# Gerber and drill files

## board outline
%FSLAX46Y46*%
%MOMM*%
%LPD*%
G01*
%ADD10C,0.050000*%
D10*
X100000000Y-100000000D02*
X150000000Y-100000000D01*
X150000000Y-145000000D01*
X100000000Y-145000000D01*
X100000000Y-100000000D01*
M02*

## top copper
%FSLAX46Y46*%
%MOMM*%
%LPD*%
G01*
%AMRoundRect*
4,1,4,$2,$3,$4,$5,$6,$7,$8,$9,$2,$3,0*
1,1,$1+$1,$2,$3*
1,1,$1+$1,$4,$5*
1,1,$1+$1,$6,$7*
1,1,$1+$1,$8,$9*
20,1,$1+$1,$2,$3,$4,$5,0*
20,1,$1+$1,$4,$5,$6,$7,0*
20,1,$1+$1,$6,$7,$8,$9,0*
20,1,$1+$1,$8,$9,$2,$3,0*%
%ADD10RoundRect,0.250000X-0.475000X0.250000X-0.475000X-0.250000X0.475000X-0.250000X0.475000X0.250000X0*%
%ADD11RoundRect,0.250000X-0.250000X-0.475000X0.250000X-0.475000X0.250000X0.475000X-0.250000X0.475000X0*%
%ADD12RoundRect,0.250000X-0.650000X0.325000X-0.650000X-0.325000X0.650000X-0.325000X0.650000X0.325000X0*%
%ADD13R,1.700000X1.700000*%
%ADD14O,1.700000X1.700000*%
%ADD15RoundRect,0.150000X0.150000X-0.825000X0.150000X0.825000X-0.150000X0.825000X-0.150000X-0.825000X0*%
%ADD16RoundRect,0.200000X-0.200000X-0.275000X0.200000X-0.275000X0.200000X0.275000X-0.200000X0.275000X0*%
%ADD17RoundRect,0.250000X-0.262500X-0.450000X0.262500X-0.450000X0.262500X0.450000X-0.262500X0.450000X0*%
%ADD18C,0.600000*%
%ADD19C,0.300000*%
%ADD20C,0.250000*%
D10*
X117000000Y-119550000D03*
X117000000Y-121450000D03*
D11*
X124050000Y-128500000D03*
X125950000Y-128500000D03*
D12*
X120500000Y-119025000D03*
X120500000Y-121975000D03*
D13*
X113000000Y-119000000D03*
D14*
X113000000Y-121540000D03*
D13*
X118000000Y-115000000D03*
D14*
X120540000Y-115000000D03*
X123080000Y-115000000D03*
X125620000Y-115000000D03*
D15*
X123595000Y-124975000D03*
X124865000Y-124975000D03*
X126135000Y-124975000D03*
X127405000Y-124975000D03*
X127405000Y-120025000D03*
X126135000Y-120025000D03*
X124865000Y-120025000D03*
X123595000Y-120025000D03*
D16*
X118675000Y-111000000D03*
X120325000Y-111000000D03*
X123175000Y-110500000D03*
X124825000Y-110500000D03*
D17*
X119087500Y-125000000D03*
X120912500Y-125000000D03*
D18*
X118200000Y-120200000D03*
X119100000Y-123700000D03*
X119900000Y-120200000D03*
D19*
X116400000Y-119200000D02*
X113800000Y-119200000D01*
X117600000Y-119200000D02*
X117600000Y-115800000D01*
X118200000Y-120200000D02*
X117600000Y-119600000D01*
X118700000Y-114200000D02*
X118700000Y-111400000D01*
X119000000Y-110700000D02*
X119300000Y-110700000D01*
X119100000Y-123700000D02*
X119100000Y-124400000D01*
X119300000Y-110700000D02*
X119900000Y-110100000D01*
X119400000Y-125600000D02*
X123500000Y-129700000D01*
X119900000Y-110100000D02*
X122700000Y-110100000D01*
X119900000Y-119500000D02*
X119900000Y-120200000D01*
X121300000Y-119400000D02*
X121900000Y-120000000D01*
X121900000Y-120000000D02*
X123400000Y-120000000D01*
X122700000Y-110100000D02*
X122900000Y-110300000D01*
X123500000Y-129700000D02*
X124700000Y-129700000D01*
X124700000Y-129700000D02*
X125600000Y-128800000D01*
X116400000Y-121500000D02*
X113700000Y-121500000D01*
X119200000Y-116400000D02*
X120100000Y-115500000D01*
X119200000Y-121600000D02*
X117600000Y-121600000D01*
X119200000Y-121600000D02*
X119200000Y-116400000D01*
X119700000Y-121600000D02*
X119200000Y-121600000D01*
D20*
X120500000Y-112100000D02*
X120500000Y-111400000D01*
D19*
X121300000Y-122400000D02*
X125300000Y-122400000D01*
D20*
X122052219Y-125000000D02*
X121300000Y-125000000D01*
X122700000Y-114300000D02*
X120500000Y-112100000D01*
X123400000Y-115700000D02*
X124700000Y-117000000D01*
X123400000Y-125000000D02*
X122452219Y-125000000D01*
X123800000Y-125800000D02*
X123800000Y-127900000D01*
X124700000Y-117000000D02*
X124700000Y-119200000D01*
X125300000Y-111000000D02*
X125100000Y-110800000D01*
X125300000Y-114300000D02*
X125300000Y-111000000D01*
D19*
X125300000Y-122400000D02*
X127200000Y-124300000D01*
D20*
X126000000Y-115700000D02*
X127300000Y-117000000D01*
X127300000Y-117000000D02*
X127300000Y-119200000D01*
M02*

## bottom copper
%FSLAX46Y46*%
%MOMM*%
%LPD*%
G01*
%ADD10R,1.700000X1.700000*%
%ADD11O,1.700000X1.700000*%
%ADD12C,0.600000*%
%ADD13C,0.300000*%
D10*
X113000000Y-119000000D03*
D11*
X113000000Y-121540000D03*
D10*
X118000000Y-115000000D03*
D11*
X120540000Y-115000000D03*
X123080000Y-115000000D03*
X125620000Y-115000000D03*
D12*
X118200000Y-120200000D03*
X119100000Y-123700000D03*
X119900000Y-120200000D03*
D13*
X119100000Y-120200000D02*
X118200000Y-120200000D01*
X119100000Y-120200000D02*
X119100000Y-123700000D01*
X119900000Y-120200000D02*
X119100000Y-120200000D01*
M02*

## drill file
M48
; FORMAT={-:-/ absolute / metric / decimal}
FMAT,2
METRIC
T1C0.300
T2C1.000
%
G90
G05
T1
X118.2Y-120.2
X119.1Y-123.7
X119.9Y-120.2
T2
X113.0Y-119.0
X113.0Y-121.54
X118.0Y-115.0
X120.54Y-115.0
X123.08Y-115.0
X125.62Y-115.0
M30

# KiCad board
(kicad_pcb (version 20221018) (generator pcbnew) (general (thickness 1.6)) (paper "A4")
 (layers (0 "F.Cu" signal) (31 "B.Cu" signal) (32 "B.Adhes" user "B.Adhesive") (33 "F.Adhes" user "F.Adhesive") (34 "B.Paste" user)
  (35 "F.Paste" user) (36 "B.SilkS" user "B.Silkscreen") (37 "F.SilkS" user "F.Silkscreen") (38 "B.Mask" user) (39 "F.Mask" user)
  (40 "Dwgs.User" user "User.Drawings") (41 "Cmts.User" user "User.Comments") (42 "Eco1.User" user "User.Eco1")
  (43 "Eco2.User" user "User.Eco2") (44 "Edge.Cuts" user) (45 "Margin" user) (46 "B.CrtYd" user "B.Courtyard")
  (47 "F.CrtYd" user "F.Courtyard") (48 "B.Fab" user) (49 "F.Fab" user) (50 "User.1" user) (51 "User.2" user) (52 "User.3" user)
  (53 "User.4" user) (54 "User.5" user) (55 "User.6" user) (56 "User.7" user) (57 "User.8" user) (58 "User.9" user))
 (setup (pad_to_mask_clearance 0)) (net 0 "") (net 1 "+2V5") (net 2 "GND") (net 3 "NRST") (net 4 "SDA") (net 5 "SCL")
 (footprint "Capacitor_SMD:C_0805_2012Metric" (layer "F.Cu") (at 117 120.5 -90)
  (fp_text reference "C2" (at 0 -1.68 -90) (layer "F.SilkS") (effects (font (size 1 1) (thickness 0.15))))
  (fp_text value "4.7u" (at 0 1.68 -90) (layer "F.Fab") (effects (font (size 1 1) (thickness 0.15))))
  (pad "1" smd roundrect (at -0.95 0 270) (size 1 1.45) (layers "F.Cu" "F.Paste" "F.Mask") (roundrect_rratio 0.25) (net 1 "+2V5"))
  (pad "2" smd roundrect (at 0.95 0 270) (size 1 1.45) (layers "F.Cu" "F.Paste" "F.Mask") (roundrect_rratio 0.25) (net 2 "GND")))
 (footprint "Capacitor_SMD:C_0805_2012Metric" (layer "F.Cu") (at 125 128.5)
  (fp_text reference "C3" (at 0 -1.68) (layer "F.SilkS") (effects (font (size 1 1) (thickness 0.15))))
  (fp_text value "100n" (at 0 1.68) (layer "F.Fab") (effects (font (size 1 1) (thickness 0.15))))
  (pad "1" smd roundrect (at -0.95 0) (size 1 1.45) (layers "F.Cu" "F.Paste" "F.Mask") (roundrect_rratio 0.25) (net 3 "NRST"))
  (pad "2" smd roundrect (at 0.95 0) (size 1 1.45) (layers "F.Cu" "F.Paste" "F.Mask") (roundrect_rratio 0.25) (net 1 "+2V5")))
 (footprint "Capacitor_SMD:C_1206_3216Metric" (layer "F.Cu") (at 120.5 120.5 -90)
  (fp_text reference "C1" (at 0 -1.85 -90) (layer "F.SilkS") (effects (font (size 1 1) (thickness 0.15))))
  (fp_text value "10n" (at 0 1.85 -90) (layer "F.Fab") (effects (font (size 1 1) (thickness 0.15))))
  (pad "1" smd roundrect (at -1.475 0 270) (size 1.15 1.8) (layers "F.Cu" "F.Paste" "F.Mask") (roundrect_rratio 0.217391) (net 1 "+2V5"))
  (pad "2" smd roundrect (at 1.475 0 270) (size 1.15 1.8) (layers "F.Cu" "F.Paste" "F.Mask") (roundrect_rratio 0.217391) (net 2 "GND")))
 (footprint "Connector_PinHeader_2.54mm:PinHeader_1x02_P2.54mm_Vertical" (layer "F.Cu") (at 113 119)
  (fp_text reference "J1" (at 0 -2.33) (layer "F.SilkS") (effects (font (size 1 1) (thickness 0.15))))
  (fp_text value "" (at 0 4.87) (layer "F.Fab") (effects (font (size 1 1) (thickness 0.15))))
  (pad "1" thru_hole rect (at 0 0) (size 1.7 1.7) (drill 1) (layers "*.Cu" "*.Mask") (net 1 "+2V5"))
  (pad "2" thru_hole oval (at 0 2.54) (size 1.7 1.7) (drill 1) (layers "*.Cu" "*.Mask") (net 2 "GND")))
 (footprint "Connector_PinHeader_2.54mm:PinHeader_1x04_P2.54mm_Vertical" (layer "F.Cu") (at 118 115 90)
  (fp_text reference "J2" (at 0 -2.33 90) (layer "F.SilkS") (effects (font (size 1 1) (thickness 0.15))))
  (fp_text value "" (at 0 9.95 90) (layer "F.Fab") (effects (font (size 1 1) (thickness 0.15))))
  (pad "1" thru_hole rect (at 0 0 90) (size 1.7 1.7) (drill 1) (layers "*.Cu" "*.Mask") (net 1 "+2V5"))
  (pad "2" thru_hole oval (at 0 2.54 90) (size 1.7 1.7) (drill 1) (layers "*.Cu" "*.Mask") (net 2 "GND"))
  (pad "3" thru_hole oval (at 0 5.08 90) (size 1.7 1.7) (drill 1) (layers "*.Cu" "*.Mask") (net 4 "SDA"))
  (pad "4" thru_hole oval (at 0 7.62 90) (size 1.7 1.7) (drill 1) (layers "*.Cu" "*.Mask") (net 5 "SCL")))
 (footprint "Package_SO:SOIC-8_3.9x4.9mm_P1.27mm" (layer "F.Cu") (at 125.5 122.5 90)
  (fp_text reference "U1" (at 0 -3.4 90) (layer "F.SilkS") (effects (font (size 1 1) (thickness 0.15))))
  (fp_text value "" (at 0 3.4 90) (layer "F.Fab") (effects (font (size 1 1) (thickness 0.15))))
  (pad "1" smd roundrect (at -2.475 -1.905 90) (size 1.95 0.6) (layers "F.Cu" "F.Paste" "F.Mask") (roundrect_rratio 0.25) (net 3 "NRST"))
  (pad "2" smd roundrect (at -2.475 -0.635 90) (size 1.95 0.6) (layers "F.Cu" "F.Paste" "F.Mask") (roundrect_rratio 0.25))
  (pad "3" smd roundrect (at -2.475 0.635 90) (size 1.95 0.6) (layers "F.Cu" "F.Paste" "F.Mask") (roundrect_rratio 0.25))
  (pad "4" smd roundrect (at -2.475 1.905 90) (size 1.95 0.6) (layers "F.Cu" "F.Paste" "F.Mask") (roundrect_rratio 0.25) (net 2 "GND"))
  (pad "5" smd roundrect (at 2.475 1.905 90) (size 1.95 0.6) (layers "F.Cu" "F.Paste" "F.Mask") (roundrect_rratio 0.25) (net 5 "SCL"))
  (pad "6" smd roundrect (at 2.475 0.635 90) (size 1.95 0.6) (layers "F.Cu" "F.Paste" "F.Mask") (roundrect_rratio 0.25))
  (pad "7" smd roundrect (at 2.475 -0.635 90) (size 1.95 0.6) (layers "F.Cu" "F.Paste" "F.Mask") (roundrect_rratio 0.25) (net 4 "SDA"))
  (pad "8" smd roundrect (at 2.475 -1.905 90) (size 1.95 0.6) (layers "F.Cu" "F.Paste" "F.Mask") (roundrect_rratio 0.25) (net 1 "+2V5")))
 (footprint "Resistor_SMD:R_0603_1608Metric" (layer "F.Cu") (at 119.5 111)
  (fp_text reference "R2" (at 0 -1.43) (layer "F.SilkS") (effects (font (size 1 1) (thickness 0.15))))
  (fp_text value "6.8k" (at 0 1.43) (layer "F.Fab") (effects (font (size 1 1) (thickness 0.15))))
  (pad "1" smd roundrect (at -0.825 0) (size 0.8 0.95) (layers "F.Cu" "F.Paste" "F.Mask") (roundrect_rratio 0.25) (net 1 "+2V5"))
  (pad "2" smd roundrect (at 0.825 0) (size 0.8 0.95) (layers "F.Cu" "F.Paste" "F.Mask") (roundrect_rratio 0.25) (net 4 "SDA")))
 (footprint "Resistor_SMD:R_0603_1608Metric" (layer "F.Cu") (at 124 110.5)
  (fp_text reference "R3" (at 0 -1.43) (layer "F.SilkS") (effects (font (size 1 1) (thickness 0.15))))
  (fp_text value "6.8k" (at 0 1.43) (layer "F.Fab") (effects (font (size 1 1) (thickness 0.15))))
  (pad "1" smd roundrect (at -0.825 0) (size 0.8 0.95) (layers "F.Cu" "F.Paste" "F.Mask") (roundrect_rratio 0.25) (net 1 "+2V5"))
  (pad "2" smd roundrect (at 0.825 0) (size 0.8 0.95) (layers "F.Cu" "F.Paste" "F.Mask") (roundrect_rratio 0.25) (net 5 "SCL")))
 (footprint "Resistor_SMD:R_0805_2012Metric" (layer "F.Cu") (at 120 125)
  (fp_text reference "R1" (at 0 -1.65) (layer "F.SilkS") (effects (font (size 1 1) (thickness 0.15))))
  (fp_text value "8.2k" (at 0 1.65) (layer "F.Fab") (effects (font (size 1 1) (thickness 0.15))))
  (pad "1" smd roundrect (at -0.9125 0) (size 1.025 1.4) (layers "F.Cu" "F.Paste" "F.Mask") (roundrect_rratio 0.243902) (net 1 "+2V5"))
  (pad "2" smd roundrect (at 0.9125 0) (size 1.025 1.4) (layers "F.Cu" "F.Paste" "F.Mask") (roundrect_rratio 0.243902) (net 3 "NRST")))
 (gr_rect (start 100 100) (end 150 145) (stroke (width 0.05) (type default)) (fill none) (layer "Edge.Cuts"))
 (segment (start 116.4 119.2) (end 113.8 119.2) (width 0.3) (layer "F.Cu") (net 1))
 (segment (start 117.6 119.2) (end 117.6 115.8) (width 0.3) (layer "F.Cu") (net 1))
 (segment (start 118.2 120.2) (end 117.6 119.6) (width 0.3) (layer "F.Cu") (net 1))
 (segment (start 118.7 114.2) (end 118.7 111.4) (width 0.3) (layer "F.Cu") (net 1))
 (segment (start 119 110.7) (end 119.3 110.7) (width 0.3) (layer "F.Cu") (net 1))
 (segment (start 119.1 123.7) (end 119.1 124.4) (width 0.3) (layer "F.Cu") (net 1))
 (segment (start 119.3 110.7) (end 119.9 110.1) (width 0.3) (layer "F.Cu") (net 1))
 (segment (start 119.4 125.6) (end 123.5 129.7) (width 0.3) (layer "F.Cu") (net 1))
 (segment (start 119.9 110.1) (end 122.7 110.1) (width 0.3) (layer "F.Cu") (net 1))
 (segment (start 119.9 119.5) (end 119.9 120.2) (width 0.3) (layer "F.Cu") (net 1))
 (segment (start 121.3 119.4) (end 121.9 120) (width 0.3) (layer "F.Cu") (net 1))
 (segment (start 121.9 120) (end 123.4 120) (width 0.3) (layer "F.Cu") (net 1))
 (segment (start 122.7 110.1) (end 122.9 110.3) (width 0.3) (layer "F.Cu") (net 1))
 (segment (start 123.5 129.7) (end 124.7 129.7) (width 0.3) (layer "F.Cu") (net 1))
 (segment (start 124.7 129.7) (end 125.6 128.8) (width 0.3) (layer "F.Cu") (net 1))
 (via (at 118.2 120.2) (size 0.6) (drill 0.3) (layers "F.Cu" "B.Cu") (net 1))
 (via (at 119.1 123.7) (size 0.6) (drill 0.3) (layers "F.Cu" "B.Cu") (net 1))
 (via (at 119.9 120.2) (size 0.6) (drill 0.3) (layers "F.Cu" "B.Cu") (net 1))
 (segment (start 116.4 121.5) (end 113.7 121.5) (width 0.3) (layer "F.Cu") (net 2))
 (segment (start 119.1 120.2) (end 118.2 120.2) (width 0.3) (layer "B.Cu") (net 1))
 (segment (start 119.1 120.2) (end 119.1 123.7) (width 0.3) (layer "B.Cu") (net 1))
 (segment (start 119.2 116.4) (end 120.1 115.5) (width 0.3) (layer "F.Cu") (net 2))
 (segment (start 119.2 121.6) (end 117.6 121.6) (width 0.3) (layer "F.Cu") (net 2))
 (segment (start 119.2 121.6) (end 119.2 116.4) (width 0.3) (layer "F.Cu") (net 2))
 (segment (start 119.7 121.6) (end 119.2 121.6) (width 0.3) (layer "F.Cu") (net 2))
 (segment (start 119.9 120.2) (end 119.1 120.2) (width 0.3) (layer "B.Cu") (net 1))
 (segment (start 120.5 112.1) (end 120.5 111.4) (width 0.25) (layer "F.Cu") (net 4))
 (segment (start 121.3 122.4) (end 125.3 122.4) (width 0.3) (layer "F.Cu") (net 2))
 (segment (start 122.052219 125) (end 121.3 125) (width 0.25) (layer "F.Cu") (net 3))
 (segment (start 122.7 114.3) (end 120.5 112.1) (width 0.25) (layer "F.Cu") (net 4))
 (segment (start 123.4 115.7) (end 124.7 117) (width 0.25) (layer "F.Cu") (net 4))
 (segment (start 123.4 125) (end 122.452219 125) (width 0.25) (layer "F.Cu") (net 3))
 (segment (start 123.8 125.8) (end 123.8 127.9) (width 0.25) (layer "F.Cu") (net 3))
 (segment (start 124.7 117) (end 124.7 119.2) (width 0.25) (layer "F.Cu") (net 4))
 (segment (start 125.3 111) (end 125.1 110.8) (width 0.25) (layer "F.Cu") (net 5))
 (segment (start 125.3 114.3) (end 125.3 111) (width 0.25) (layer "F.Cu") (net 5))
 (segment (start 125.3 122.4) (end 127.2 124.3) (width 0.3) (layer "F.Cu") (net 2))
 (segment (start 126 115.7) (end 127.3 117) (width 0.25) (layer "F.Cu") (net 5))
 (segment (start 127.3 117) (end 127.3 119.2) (width 0.25) (layer "F.Cu") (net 5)))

